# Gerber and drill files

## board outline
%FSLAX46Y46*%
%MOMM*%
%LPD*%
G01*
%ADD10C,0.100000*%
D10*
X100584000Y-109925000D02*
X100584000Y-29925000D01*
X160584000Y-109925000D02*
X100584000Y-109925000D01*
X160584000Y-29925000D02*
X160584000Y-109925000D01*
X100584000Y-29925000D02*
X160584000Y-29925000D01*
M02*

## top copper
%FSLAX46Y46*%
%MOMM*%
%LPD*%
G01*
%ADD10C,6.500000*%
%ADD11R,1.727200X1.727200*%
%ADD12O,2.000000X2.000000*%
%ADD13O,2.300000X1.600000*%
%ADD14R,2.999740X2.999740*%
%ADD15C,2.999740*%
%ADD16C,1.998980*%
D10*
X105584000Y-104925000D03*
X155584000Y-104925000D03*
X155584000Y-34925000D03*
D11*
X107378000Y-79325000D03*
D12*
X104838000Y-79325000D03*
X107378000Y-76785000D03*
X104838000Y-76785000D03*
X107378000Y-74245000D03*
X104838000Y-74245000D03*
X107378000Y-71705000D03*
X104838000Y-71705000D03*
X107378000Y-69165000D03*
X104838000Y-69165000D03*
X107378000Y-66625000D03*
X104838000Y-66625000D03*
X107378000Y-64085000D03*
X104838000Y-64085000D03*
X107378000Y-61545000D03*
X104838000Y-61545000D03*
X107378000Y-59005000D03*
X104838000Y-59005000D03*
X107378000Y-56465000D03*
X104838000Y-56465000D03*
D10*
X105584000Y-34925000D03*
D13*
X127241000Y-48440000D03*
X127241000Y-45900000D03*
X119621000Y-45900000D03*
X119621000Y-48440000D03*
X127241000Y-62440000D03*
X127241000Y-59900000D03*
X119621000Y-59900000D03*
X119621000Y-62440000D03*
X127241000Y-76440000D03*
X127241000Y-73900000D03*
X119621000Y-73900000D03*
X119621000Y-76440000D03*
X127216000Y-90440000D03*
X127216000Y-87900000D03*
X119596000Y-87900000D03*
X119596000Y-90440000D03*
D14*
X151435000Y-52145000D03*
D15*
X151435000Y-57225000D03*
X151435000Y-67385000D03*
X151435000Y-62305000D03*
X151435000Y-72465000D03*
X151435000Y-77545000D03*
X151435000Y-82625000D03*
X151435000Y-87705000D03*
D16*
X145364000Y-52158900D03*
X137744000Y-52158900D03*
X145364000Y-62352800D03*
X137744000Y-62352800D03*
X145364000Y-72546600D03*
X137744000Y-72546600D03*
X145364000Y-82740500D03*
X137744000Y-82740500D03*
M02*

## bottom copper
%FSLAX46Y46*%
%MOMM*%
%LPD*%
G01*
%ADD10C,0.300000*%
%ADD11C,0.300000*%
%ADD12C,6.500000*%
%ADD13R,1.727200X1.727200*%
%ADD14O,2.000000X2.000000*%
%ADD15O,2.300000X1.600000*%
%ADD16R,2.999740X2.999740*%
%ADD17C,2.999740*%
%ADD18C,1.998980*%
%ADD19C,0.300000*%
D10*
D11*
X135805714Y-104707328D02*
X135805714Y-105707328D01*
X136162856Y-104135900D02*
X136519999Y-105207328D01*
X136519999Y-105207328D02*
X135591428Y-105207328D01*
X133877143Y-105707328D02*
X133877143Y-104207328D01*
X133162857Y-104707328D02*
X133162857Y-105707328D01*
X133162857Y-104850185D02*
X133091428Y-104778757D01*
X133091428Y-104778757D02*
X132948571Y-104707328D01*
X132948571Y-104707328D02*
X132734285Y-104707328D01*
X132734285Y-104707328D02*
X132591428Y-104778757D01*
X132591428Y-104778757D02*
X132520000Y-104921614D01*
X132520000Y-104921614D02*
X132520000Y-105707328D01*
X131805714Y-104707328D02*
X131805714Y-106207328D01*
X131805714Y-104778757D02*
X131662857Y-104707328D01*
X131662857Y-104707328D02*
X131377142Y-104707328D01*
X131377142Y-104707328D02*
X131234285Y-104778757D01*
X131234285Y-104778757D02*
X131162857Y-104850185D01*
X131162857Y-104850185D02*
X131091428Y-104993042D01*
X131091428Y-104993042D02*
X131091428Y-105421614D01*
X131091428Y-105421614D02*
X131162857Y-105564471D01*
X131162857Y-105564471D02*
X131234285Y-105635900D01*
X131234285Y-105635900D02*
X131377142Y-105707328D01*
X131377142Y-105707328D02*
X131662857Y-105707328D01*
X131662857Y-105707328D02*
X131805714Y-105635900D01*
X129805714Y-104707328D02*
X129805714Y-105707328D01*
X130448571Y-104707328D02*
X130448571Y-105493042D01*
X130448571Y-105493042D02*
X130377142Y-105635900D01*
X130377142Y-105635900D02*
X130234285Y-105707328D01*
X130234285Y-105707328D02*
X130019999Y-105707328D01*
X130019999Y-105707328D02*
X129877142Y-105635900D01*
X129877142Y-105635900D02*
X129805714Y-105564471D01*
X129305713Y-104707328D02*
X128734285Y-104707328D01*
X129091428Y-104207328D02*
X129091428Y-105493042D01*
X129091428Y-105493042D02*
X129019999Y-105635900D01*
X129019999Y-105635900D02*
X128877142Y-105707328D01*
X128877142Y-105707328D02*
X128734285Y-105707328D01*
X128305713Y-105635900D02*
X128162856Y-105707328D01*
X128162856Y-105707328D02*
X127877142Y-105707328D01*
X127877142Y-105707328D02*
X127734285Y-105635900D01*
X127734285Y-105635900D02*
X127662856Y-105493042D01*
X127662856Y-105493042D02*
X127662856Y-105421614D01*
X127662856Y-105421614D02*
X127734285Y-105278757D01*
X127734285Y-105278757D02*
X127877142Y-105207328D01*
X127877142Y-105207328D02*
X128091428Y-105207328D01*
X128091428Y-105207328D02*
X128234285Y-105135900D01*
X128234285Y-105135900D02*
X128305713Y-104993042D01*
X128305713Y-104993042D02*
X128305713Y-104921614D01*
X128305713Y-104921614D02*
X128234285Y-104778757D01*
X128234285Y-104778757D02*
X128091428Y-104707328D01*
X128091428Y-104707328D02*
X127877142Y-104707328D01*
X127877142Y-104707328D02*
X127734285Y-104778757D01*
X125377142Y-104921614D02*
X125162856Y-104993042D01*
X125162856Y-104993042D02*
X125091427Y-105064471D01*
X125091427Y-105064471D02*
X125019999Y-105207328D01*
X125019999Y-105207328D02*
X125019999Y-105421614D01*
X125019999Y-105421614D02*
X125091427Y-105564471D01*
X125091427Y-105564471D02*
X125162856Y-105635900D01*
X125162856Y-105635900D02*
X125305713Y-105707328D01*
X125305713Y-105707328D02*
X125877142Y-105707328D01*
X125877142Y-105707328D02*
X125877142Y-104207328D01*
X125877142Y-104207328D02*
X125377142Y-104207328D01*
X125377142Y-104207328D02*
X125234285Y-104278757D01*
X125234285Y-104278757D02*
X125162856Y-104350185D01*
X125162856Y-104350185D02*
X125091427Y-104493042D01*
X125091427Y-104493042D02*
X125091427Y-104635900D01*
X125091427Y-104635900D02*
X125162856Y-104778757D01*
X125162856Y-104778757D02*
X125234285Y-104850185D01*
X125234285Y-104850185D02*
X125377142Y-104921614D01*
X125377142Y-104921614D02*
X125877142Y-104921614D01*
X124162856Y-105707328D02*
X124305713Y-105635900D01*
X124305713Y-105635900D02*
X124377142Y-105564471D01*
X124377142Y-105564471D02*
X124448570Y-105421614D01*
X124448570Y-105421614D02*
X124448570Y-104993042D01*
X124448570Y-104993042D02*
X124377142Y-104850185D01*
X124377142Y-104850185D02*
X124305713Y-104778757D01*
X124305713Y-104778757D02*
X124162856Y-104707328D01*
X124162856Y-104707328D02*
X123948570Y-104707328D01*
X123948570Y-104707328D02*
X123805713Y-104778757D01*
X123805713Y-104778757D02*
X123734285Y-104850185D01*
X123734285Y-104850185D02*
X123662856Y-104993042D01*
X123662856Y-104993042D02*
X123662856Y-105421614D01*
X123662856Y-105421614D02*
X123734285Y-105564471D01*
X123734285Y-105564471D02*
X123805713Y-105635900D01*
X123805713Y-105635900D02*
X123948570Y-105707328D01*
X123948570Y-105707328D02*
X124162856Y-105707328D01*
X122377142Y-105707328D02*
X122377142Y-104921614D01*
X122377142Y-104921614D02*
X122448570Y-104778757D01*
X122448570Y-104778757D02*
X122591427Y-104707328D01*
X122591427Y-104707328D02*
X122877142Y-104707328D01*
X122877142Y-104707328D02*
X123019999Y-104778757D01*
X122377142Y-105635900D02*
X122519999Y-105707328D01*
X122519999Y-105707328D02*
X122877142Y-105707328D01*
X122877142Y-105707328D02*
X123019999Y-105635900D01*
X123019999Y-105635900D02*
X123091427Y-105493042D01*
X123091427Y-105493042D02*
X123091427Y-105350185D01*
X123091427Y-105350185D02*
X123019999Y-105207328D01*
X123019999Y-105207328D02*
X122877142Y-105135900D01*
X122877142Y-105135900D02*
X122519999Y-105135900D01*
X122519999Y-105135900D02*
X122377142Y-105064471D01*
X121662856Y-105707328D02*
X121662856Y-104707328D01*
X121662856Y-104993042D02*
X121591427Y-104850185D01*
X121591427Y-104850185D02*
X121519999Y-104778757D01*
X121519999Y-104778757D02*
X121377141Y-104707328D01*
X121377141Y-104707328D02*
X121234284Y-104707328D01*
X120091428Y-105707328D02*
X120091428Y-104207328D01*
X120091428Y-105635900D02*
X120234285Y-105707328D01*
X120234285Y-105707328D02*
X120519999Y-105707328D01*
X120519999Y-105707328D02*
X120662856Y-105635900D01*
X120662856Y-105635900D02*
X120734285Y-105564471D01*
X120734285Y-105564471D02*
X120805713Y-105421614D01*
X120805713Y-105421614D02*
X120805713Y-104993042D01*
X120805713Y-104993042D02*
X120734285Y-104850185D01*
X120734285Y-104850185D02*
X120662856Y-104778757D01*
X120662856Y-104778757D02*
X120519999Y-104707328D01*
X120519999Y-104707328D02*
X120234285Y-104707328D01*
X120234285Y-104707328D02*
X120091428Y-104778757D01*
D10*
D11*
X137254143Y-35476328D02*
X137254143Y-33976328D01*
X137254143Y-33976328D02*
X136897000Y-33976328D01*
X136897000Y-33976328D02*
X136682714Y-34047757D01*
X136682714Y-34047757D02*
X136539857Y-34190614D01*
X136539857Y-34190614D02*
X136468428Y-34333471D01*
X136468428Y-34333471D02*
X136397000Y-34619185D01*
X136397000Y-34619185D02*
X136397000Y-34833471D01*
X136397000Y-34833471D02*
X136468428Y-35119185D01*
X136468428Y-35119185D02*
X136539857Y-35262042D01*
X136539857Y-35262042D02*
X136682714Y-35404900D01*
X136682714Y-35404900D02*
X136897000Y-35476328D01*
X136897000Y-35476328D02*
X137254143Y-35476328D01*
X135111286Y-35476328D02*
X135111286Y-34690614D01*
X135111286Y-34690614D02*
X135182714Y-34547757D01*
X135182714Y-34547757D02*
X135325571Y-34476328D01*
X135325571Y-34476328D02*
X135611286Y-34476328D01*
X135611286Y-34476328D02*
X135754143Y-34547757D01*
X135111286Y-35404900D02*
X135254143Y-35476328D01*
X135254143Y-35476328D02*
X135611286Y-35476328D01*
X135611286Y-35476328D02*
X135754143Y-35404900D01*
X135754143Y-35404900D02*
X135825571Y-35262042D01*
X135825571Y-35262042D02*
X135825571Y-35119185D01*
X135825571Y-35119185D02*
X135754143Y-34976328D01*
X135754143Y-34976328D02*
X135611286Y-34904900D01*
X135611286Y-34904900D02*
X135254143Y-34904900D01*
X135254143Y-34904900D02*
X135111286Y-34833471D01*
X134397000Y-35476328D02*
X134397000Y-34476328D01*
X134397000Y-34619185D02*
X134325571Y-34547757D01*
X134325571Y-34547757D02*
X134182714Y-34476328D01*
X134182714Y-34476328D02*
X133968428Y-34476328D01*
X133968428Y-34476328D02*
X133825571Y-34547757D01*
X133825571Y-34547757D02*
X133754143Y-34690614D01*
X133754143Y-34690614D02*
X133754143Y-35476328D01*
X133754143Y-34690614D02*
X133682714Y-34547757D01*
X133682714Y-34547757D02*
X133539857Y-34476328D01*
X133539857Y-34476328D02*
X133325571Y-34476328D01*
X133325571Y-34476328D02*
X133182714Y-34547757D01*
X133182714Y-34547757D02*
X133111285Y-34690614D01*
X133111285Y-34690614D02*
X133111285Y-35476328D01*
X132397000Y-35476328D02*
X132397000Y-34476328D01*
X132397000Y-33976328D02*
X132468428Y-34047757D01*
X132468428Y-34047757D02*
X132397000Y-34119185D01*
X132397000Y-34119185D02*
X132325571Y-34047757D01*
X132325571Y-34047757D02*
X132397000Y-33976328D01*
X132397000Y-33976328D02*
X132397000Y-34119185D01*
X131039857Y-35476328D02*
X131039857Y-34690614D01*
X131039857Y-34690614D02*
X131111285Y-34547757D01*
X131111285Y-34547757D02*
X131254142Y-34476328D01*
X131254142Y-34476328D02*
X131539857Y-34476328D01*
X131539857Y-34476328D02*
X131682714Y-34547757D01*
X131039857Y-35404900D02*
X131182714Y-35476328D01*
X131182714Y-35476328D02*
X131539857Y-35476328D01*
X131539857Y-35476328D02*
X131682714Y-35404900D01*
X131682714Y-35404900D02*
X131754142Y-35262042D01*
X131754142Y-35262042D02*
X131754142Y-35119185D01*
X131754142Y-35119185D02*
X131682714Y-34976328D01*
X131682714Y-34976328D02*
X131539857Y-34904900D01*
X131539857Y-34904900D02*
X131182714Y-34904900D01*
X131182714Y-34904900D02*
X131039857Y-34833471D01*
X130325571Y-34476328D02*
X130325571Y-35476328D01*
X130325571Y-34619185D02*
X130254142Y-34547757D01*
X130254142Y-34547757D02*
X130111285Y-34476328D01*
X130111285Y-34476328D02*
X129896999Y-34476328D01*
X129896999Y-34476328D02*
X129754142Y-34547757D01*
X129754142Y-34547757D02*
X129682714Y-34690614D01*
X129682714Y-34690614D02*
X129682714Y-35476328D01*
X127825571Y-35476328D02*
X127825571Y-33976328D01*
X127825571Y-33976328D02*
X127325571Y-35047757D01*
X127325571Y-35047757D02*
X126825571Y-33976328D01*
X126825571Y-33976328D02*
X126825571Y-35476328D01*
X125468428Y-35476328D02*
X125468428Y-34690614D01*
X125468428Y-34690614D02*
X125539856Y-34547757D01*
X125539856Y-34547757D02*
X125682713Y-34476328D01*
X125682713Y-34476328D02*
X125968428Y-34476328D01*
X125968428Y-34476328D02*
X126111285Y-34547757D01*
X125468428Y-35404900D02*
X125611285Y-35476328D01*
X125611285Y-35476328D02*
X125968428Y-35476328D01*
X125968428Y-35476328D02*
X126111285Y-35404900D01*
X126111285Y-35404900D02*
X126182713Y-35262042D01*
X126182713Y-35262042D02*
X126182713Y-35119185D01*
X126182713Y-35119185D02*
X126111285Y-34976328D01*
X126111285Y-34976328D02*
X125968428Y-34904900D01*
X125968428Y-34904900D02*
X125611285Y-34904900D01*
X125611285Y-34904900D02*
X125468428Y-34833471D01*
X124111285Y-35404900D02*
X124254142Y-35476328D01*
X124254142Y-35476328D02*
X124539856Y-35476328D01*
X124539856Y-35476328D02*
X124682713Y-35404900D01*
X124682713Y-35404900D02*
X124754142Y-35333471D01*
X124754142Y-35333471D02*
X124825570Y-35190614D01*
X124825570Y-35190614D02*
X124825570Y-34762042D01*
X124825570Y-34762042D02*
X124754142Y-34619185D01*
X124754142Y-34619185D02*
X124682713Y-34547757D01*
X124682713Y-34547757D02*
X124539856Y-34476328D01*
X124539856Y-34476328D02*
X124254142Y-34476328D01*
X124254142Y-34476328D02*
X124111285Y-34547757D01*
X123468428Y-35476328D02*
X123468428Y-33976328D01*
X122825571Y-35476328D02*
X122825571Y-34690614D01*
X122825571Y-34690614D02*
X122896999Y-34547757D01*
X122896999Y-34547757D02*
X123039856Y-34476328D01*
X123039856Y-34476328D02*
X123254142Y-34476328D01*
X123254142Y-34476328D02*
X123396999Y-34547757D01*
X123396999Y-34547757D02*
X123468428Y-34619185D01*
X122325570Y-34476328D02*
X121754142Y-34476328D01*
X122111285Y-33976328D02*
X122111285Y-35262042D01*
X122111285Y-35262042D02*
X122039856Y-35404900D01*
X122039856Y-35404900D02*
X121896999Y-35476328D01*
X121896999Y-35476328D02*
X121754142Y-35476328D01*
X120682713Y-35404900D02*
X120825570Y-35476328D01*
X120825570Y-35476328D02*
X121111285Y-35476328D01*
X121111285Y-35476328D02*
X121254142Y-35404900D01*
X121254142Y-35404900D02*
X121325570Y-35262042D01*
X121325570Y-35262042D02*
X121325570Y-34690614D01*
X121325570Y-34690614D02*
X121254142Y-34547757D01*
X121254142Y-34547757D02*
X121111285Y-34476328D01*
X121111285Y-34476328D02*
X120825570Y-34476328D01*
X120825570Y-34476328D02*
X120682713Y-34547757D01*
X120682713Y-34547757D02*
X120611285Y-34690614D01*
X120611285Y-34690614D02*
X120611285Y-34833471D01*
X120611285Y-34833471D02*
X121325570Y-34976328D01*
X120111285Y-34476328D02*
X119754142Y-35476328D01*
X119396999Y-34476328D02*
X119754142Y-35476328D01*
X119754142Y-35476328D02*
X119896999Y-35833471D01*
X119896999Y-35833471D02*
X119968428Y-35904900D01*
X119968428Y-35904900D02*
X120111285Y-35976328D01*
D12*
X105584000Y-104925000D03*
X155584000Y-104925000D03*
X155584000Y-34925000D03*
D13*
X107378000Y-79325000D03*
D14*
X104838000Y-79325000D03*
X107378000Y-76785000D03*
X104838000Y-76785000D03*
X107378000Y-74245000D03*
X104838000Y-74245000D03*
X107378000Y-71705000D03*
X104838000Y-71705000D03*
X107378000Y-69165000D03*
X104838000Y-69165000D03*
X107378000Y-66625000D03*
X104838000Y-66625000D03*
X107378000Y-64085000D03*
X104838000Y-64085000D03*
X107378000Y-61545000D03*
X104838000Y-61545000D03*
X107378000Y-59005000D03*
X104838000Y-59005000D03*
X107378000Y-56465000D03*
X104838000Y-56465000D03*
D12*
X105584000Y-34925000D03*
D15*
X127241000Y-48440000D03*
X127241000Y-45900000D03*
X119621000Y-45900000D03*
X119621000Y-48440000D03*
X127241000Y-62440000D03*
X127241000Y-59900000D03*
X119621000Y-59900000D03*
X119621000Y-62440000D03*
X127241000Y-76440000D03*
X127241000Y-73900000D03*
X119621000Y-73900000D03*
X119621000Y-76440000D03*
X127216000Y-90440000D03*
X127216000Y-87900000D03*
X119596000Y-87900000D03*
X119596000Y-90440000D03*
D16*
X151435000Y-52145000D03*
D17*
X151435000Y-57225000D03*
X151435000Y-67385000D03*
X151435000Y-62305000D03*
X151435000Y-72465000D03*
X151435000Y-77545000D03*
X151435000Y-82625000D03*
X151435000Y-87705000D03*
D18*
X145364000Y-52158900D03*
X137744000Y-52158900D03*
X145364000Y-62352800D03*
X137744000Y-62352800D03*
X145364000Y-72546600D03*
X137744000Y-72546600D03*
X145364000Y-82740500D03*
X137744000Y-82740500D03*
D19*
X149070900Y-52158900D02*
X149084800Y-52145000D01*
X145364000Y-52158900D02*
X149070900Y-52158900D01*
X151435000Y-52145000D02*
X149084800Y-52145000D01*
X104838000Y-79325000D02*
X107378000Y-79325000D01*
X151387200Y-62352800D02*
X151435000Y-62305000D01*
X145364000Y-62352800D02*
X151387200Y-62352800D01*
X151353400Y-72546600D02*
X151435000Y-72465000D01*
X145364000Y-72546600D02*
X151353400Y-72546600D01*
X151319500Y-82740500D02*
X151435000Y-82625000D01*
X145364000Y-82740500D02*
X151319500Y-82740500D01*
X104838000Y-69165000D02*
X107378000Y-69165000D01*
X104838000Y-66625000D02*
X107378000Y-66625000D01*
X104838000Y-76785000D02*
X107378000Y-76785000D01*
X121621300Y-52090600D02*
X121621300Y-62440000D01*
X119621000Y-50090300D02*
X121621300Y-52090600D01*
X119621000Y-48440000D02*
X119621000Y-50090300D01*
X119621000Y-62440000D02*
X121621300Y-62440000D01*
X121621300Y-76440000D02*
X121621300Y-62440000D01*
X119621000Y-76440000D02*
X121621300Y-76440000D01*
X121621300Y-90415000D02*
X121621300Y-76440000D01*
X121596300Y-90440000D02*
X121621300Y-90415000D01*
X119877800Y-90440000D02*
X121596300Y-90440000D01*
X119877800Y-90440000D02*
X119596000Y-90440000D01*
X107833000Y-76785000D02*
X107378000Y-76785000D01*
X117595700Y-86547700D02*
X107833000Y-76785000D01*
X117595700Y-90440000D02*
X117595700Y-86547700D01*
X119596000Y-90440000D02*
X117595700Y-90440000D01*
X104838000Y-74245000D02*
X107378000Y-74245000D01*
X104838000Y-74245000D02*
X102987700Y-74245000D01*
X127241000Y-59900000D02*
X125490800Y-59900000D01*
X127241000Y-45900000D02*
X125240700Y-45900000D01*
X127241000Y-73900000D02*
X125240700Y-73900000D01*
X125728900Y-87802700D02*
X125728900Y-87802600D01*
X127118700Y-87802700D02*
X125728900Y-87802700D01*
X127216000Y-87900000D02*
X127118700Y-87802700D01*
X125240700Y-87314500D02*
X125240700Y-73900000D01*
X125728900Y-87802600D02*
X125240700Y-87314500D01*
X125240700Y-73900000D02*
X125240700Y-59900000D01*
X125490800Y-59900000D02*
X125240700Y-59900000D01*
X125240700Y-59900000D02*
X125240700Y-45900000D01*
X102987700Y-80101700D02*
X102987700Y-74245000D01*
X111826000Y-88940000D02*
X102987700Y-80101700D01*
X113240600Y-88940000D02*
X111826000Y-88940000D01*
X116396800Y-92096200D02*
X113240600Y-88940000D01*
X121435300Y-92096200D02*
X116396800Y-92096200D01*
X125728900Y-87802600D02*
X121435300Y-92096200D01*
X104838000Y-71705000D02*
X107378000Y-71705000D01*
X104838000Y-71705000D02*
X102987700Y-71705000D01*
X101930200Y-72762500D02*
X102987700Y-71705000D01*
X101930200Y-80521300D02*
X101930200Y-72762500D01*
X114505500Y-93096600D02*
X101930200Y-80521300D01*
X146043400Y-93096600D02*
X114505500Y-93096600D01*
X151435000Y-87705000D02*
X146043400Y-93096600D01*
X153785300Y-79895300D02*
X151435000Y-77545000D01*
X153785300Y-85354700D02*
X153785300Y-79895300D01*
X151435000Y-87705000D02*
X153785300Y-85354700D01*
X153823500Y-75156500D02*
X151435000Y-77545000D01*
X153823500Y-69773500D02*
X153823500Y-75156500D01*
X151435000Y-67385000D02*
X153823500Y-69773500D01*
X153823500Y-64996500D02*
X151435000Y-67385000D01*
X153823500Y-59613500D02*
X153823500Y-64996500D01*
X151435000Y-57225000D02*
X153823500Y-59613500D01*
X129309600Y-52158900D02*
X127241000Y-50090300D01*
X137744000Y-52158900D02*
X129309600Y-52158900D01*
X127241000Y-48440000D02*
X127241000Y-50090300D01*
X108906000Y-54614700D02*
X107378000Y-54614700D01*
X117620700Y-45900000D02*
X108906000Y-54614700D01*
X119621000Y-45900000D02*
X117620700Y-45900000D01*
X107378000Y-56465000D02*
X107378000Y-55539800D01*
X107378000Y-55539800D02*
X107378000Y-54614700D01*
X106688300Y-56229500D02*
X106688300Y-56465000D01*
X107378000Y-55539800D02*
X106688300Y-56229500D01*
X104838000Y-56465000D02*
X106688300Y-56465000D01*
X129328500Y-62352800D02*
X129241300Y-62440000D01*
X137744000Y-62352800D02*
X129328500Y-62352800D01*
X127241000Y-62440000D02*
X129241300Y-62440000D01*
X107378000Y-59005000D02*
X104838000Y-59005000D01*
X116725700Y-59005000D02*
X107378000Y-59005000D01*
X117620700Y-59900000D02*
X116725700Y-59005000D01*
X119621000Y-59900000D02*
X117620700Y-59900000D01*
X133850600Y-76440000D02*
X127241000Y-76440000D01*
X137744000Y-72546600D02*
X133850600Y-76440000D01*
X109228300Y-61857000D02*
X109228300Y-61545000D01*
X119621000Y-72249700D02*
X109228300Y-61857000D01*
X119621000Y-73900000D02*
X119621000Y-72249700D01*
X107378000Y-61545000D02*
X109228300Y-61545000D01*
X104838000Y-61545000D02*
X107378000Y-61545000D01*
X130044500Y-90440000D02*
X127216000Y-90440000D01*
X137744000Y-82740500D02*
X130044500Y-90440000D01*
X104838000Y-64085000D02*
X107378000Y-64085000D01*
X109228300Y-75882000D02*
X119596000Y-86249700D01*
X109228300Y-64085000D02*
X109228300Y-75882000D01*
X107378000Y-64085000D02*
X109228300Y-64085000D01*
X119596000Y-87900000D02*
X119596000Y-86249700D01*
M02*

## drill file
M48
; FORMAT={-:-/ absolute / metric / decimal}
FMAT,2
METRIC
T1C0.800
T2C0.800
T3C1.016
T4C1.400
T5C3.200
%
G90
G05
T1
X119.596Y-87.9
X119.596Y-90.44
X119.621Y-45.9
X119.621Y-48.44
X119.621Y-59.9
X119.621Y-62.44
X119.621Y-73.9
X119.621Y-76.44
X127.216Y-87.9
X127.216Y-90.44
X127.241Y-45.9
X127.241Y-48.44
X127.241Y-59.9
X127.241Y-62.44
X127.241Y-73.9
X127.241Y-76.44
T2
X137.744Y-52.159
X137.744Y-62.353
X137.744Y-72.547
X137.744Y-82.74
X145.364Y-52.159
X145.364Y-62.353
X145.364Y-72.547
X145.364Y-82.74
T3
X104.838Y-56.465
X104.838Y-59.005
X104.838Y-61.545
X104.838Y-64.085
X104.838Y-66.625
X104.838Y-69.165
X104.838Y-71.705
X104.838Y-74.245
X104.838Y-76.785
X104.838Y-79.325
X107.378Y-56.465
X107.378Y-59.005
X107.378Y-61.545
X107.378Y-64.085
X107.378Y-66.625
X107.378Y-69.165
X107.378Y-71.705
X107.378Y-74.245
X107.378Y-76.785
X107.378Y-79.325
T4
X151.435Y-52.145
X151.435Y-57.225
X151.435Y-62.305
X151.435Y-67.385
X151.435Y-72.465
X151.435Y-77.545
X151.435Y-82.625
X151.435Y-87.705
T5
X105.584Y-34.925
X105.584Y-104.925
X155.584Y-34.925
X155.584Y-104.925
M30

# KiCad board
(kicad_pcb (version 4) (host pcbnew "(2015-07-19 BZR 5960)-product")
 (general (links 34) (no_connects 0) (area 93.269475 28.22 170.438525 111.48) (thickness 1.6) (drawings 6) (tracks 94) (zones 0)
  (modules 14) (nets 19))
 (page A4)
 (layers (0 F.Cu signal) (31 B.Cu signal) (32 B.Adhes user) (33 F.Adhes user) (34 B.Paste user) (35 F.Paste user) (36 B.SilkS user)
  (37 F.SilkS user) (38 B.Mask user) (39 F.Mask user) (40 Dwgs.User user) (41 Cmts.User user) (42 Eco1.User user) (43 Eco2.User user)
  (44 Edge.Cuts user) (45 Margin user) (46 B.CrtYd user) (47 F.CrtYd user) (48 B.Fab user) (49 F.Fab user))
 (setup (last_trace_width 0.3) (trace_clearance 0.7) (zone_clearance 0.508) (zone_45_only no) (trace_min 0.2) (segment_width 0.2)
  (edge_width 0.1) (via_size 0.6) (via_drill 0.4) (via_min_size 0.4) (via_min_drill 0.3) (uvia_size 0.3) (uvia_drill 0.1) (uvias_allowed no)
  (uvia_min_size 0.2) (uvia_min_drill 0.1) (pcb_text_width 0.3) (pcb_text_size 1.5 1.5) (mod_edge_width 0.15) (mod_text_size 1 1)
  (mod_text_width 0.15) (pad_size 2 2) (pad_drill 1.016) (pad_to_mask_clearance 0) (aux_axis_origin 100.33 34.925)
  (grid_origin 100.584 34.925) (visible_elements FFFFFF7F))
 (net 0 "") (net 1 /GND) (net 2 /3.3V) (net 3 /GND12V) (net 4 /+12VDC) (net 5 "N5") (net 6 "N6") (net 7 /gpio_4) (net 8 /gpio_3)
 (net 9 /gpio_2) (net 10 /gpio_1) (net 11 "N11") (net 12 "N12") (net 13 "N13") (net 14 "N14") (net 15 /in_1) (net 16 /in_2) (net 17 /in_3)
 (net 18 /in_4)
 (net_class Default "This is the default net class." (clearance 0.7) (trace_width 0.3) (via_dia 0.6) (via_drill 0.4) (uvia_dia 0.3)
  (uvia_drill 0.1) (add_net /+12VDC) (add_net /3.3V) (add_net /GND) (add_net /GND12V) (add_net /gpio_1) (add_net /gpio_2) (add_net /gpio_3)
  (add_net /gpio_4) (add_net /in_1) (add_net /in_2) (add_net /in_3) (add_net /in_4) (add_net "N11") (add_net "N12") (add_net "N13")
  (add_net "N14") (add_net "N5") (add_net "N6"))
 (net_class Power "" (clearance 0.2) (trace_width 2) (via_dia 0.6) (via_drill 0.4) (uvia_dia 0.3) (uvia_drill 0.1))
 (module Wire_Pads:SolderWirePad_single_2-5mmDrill (layer F.Cu) (at 105.584 104.925)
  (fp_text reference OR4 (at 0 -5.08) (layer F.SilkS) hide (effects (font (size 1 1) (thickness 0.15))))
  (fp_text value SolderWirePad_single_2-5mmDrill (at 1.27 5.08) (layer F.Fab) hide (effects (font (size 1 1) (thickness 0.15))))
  (pad 1 thru_hole circle (at 0 0) (size 6.5 6.5) (drill 3.2) (layers *.Cu *.Mask F.SilkS)))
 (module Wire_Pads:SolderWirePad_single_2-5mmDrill (layer F.Cu) (at 155.584 104.925)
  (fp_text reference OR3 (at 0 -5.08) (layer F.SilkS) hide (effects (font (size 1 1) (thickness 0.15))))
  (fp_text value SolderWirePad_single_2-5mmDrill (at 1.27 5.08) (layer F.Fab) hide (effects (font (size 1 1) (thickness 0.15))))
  (pad 1 thru_hole circle (at 0 0) (size 6.5 6.5) (drill 3.2) (layers *.Cu *.Mask F.SilkS)))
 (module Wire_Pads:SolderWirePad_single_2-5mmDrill (layer F.Cu) (at 155.584 34.925)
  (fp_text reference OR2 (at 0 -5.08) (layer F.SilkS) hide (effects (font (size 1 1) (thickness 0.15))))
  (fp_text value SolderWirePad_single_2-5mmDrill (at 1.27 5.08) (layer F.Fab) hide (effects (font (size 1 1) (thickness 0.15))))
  (pad 1 thru_hole circle (at 0 0) (size 6.5 6.5) (drill 3.2) (layers *.Cu *.Mask F.SilkS)))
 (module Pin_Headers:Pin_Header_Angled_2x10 (layer F.Cu) (at 107.378 79.325 180)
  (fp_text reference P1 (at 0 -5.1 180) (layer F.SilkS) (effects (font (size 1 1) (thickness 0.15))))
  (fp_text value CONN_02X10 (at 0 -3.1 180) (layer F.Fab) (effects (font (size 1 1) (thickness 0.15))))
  (pad 1 thru_hole rect (at 0 0 180) (size 1.7272 1.7272) (drill 1.016) (layers *.Cu *.Mask F.SilkS) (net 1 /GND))
  (pad 2 thru_hole oval (at 2.54 0 180) (size 2 2) (drill 1.016) (layers *.Cu *.Mask F.SilkS) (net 1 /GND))
  (pad 3 thru_hole oval (at 0 2.54 180) (size 2 2) (drill 1.016) (layers *.Cu *.Mask F.SilkS) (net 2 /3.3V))
  (pad 4 thru_hole oval (at 2.54 2.54 180) (size 2 2) (drill 1.016) (layers *.Cu *.Mask F.SilkS) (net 2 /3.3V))
  (pad 5 thru_hole oval (at 0 5.08 180) (size 2 2) (drill 1.016) (layers *.Cu *.Mask F.SilkS) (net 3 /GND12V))
  (pad 6 thru_hole oval (at 2.54 5.08 180) (size 2 2) (drill 1.016) (layers *.Cu *.Mask F.SilkS) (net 3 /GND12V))
  (pad 7 thru_hole oval (at 0 7.62 180) (size 2 2) (drill 1.016) (layers *.Cu *.Mask F.SilkS) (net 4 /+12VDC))
  (pad 8 thru_hole oval (at 2.54 7.62 180) (size 2 2) (drill 1.016) (layers *.Cu *.Mask F.SilkS) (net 4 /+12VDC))
  (pad 9 thru_hole oval (at 0 10.16 180) (size 2 2) (drill 1.016) (layers *.Cu *.Mask F.SilkS) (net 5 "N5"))
  (pad 10 thru_hole oval (at 2.54 10.16 180) (size 2 2) (drill 1.016) (layers *.Cu *.Mask F.SilkS) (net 5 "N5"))
  (pad 11 thru_hole oval (at 0 12.7 180) (size 2 2) (drill 1.016) (layers *.Cu *.Mask F.SilkS) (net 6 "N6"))
  (pad 12 thru_hole oval (at 2.54 12.7 180) (size 2 2) (drill 1.016) (layers *.Cu *.Mask F.SilkS) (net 6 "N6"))
  (pad 13 thru_hole oval (at 0 15.24 180) (size 2 2) (drill 1.016) (layers *.Cu *.Mask F.SilkS) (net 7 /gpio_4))
  (pad 14 thru_hole oval (at 2.54 15.24 180) (size 2 2) (drill 1.016) (layers *.Cu *.Mask F.SilkS) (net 7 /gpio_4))
  (pad 15 thru_hole oval (at 0 17.78 180) (size 2 2) (drill 1.016) (layers *.Cu *.Mask F.SilkS) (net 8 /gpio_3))
  (pad 16 thru_hole oval (at 2.54 17.78 180) (size 2 2) (drill 1.016) (layers *.Cu *.Mask F.SilkS) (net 8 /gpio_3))
  (pad 17 thru_hole oval (at 0 20.32 180) (size 2 2) (drill 1.016) (layers *.Cu *.Mask F.SilkS) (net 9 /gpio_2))
  (pad 18 thru_hole oval (at 2.54 20.32 180) (size 2 2) (drill 1.016) (layers *.Cu *.Mask F.SilkS) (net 9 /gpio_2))
  (pad 19 thru_hole oval (at 0 22.86 180) (size 2 2) (drill 1.016) (layers *.Cu *.Mask F.SilkS) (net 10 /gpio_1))
  (pad 20 thru_hole oval (at 2.54 22.86 180) (size 2 2) (drill 1.016) (layers *.Cu *.Mask F.SilkS) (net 10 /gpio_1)))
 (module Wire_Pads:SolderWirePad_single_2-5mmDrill (layer F.Cu) (at 105.584 34.925)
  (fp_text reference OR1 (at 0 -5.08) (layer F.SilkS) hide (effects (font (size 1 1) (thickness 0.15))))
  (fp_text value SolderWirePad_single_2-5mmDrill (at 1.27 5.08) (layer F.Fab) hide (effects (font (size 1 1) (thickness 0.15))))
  (pad 1 thru_hole circle (at 0 0) (size 6.5 6.5) (drill 3.2) (layers *.Cu *.Mask F.SilkS)))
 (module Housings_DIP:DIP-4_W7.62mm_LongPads (layer F.Cu) (at 127.241 48.44 180)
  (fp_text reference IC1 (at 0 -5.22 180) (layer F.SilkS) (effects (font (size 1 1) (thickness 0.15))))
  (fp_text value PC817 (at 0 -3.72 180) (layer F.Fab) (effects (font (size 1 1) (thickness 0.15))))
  (pad 1 thru_hole oval (at 0 0 180) (size 2.3 1.6) (drill 0.8) (layers *.Cu *.Mask F.SilkS) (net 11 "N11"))
  (pad 2 thru_hole oval (at 0 2.54 180) (size 2.3 1.6) (drill 0.8) (layers *.Cu *.Mask F.SilkS) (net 3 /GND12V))
  (pad 3 thru_hole oval (at 7.62 2.54 180) (size 2.3 1.6) (drill 0.8) (layers *.Cu *.Mask F.SilkS) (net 10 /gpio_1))
  (pad 4 thru_hole oval (at 7.62 0 180) (size 2.3 1.6) (drill 0.8) (layers *.Cu *.Mask F.SilkS) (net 2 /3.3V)))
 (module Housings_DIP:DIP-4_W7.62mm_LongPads (layer F.Cu) (at 127.241 62.44 180)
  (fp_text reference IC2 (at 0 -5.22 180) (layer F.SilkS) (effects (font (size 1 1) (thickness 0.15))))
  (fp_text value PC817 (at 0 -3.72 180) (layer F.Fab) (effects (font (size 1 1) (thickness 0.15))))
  (pad 1 thru_hole oval (at 0 0 180) (size 2.3 1.6) (drill 0.8) (layers *.Cu *.Mask F.SilkS) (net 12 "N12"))
  (pad 2 thru_hole oval (at 0 2.54 180) (size 2.3 1.6) (drill 0.8) (layers *.Cu *.Mask F.SilkS) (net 3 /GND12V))
  (pad 3 thru_hole oval (at 7.62 2.54 180) (size 2.3 1.6) (drill 0.8) (layers *.Cu *.Mask F.SilkS) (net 9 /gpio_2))
  (pad 4 thru_hole oval (at 7.62 0 180) (size 2.3 1.6) (drill 0.8) (layers *.Cu *.Mask F.SilkS) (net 2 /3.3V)))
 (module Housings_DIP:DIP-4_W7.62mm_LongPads (layer F.Cu) (at 127.241 76.44 180)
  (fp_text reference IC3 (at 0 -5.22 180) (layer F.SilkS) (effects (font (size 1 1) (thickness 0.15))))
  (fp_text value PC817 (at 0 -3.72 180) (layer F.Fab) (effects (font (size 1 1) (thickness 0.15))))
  (pad 1 thru_hole oval (at 0 0 180) (size 2.3 1.6) (drill 0.8) (layers *.Cu *.Mask F.SilkS) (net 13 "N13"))
  (pad 2 thru_hole oval (at 0 2.54 180) (size 2.3 1.6) (drill 0.8) (layers *.Cu *.Mask F.SilkS) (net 3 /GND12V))
  (pad 3 thru_hole oval (at 7.62 2.54 180) (size 2.3 1.6) (drill 0.8) (layers *.Cu *.Mask F.SilkS) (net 8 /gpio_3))
  (pad 4 thru_hole oval (at 7.62 0 180) (size 2.3 1.6) (drill 0.8) (layers *.Cu *.Mask F.SilkS) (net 2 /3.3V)))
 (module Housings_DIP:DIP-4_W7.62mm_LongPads (layer F.Cu) (at 127.216 90.44 180)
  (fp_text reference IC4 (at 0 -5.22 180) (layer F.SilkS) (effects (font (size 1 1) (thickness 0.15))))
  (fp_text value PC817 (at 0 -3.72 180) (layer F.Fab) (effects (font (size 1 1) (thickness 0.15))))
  (pad 1 thru_hole oval (at 0 0 180) (size 2.3 1.6) (drill 0.8) (layers *.Cu *.Mask F.SilkS) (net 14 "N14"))
  (pad 2 thru_hole oval (at 0 2.54 180) (size 2.3 1.6) (drill 0.8) (layers *.Cu *.Mask F.SilkS) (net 3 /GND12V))
  (pad 3 thru_hole oval (at 7.62 2.54 180) (size 2.3 1.6) (drill 0.8) (layers *.Cu *.Mask F.SilkS) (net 7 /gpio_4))
  (pad 4 thru_hole oval (at 7.62 0 180) (size 2.3 1.6) (drill 0.8) (layers *.Cu *.Mask F.SilkS) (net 2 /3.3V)))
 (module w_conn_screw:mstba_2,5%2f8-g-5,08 (layer F.Cu) (at 151.435 69.925 270)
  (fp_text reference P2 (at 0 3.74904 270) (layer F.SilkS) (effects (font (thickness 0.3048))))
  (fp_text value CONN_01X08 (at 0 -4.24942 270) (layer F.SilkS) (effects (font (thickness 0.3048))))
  (pad 1 thru_hole rect (at -17.78 0 270) (size 2.99974 2.99974) (drill 1.39954) (layers *.Cu *.Mask F.SilkS) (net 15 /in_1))
  (pad 2 thru_hole circle (at -12.7 0 270) (size 2.99974 2.99974) (drill 1.39954) (layers *.Cu *.Mask F.SilkS) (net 4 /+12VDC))
  (pad 4 thru_hole circle (at -2.54 0 270) (size 2.99974 2.99974) (drill 1.39954) (layers *.Cu *.Mask F.SilkS) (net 4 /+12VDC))
  (pad 3 thru_hole circle (at -7.62 0 270) (size 2.99974 2.99974) (drill 1.39954) (layers *.Cu *.Mask F.SilkS) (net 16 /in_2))
  (pad 5 thru_hole circle (at 2.54 0 270) (size 2.99974 2.99974) (drill 1.39954) (layers *.Cu *.Mask F.SilkS) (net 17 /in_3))
  (pad 6 thru_hole circle (at 7.62 0 270) (size 2.99974 2.99974) (drill 1.39954) (layers *.Cu *.Mask F.SilkS) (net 4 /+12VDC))
  (pad 7 thru_hole circle (at 12.7 0 270) (size 2.99974 2.99974) (drill 1.39954) (layers *.Cu *.Mask F.SilkS) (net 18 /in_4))
  (pad 8 thru_hole circle (at 17.78 0 270) (size 2.99974 2.99974) (drill 1.39954) (layers *.Cu *.Mask F.SilkS) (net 4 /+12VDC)))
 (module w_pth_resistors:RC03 (layer F.Cu) (at 141.554 52.1589 180) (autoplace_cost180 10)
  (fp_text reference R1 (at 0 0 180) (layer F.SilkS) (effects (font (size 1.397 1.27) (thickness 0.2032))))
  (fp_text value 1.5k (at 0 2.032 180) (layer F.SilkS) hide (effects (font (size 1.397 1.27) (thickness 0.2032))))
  (pad 1 thru_hole circle (at -3.81 0 180) (size 1.99898 1.99898) (drill 0.8001) (layers *.Cu *.Mask F.SilkS) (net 15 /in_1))
  (pad 2 thru_hole circle (at 3.81 0 180) (size 1.99898 1.99898) (drill 0.8001) (layers *.Cu *.Mask F.SilkS) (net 11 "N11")))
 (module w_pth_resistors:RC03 (layer F.Cu) (at 141.554 62.3528 180) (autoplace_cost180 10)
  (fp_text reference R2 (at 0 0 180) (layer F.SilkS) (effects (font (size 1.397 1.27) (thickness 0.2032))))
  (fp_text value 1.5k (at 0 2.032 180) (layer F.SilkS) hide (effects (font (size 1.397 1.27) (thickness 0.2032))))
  (pad 1 thru_hole circle (at -3.81 0 180) (size 1.99898 1.99898) (drill 0.8001) (layers *.Cu *.Mask F.SilkS) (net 16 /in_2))
  (pad 2 thru_hole circle (at 3.81 0 180) (size 1.99898 1.99898) (drill 0.8001) (layers *.Cu *.Mask F.SilkS) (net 12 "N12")))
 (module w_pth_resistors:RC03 (layer F.Cu) (at 141.554 72.5466 180) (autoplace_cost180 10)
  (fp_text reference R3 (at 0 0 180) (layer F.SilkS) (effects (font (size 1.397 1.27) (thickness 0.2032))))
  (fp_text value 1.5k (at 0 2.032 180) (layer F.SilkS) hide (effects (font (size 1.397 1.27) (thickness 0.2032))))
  (pad 1 thru_hole circle (at -3.81 0 180) (size 1.99898 1.99898) (drill 0.8001) (layers *.Cu *.Mask F.SilkS) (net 17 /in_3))
  (pad 2 thru_hole circle (at 3.81 0 180) (size 1.99898 1.99898) (drill 0.8001) (layers *.Cu *.Mask F.SilkS) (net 13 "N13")))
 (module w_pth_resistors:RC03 (layer F.Cu) (at 141.554 82.7405 180) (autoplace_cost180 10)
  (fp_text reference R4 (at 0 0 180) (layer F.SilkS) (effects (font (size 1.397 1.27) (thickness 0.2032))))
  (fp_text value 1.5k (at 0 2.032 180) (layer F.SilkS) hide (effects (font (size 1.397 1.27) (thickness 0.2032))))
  (pad 1 thru_hole circle (at -3.81 0 180) (size 1.99898 1.99898) (drill 0.8001) (layers *.Cu *.Mask F.SilkS) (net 18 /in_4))
  (pad 2 thru_hole circle (at 3.81 0 180) (size 1.99898 1.99898) (drill 0.8001) (layers *.Cu *.Mask F.SilkS) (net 14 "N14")))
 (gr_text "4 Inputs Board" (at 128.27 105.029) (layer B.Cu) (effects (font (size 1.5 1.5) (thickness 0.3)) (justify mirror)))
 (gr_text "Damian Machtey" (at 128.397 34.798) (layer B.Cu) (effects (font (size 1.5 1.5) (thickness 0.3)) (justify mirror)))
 (gr_line (start 100.584 109.925) (end 100.584 29.925) (angle 90) (layer Edge.Cuts) (width 0.1))
 (gr_line (start 160.584 109.925) (end 100.584 109.925) (angle 90) (layer Edge.Cuts) (width 0.1))
 (gr_line (start 160.584 29.925) (end 160.584 109.925) (angle 90) (layer Edge.Cuts) (width 0.1))
 (gr_line (start 100.584 29.925) (end 160.584 29.925) (angle 90) (layer Edge.Cuts) (width 0.1))
 (segment (start 149.0709 52.1589) (end 149.0848 52.145) (width 0.3) (layer B.Cu) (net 15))
 (segment (start 145.364 52.1589) (end 149.0709 52.1589) (width 0.3) (layer B.Cu) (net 15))
 (segment (start 151.435 52.145) (end 149.0848 52.145) (width 0.3) (layer B.Cu) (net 15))
 (segment (start 104.838 79.325) (end 107.378 79.325) (width 0.3) (layer B.Cu) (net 1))
 (segment (start 151.3872 62.3528) (end 151.435 62.305) (width 0.3) (layer B.Cu) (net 16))
 (segment (start 145.364 62.3528) (end 151.3872 62.3528) (width 0.3) (layer B.Cu) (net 16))
 (segment (start 151.3534 72.5466) (end 151.435 72.465) (width 0.3) (layer B.Cu) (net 17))
 (segment (start 145.364 72.5466) (end 151.3534 72.5466) (width 0.3) (layer B.Cu) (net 17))
 (segment (start 151.3195 82.7405) (end 151.435 82.625) (width 0.3) (layer B.Cu) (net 18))
 (segment (start 145.364 82.7405) (end 151.3195 82.7405) (width 0.3) (layer B.Cu) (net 18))
 (segment (start 104.838 69.165) (end 107.378 69.165) (width 0.3) (layer B.Cu) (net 5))
 (segment (start 104.838 66.625) (end 107.378 66.625) (width 0.3) (layer B.Cu) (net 6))
 (segment (start 104.838 76.785) (end 107.378 76.785) (width 0.3) (layer B.Cu) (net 2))
 (segment (start 121.6213 52.0906) (end 121.6213 62.44) (width 0.3) (layer B.Cu) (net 2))
 (segment (start 119.621 50.0903) (end 121.6213 52.0906) (width 0.3) (layer B.Cu) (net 2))
 (segment (start 119.621 48.44) (end 119.621 50.0903) (width 0.3) (layer B.Cu) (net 2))
 (segment (start 119.621 62.44) (end 121.6213 62.44) (width 0.3) (layer B.Cu) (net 2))
 (segment (start 121.6213 76.44) (end 121.6213 62.44) (width 0.3) (layer B.Cu) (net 2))
 (segment (start 119.621 76.44) (end 121.6213 76.44) (width 0.3) (layer B.Cu) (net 2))
 (segment (start 121.6213 90.415) (end 121.6213 76.44) (width 0.3) (layer B.Cu) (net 2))
 (segment (start 121.5963 90.44) (end 121.6213 90.415) (width 0.3) (layer B.Cu) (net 2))
 (segment (start 119.8778 90.44) (end 121.5963 90.44) (width 0.3) (layer B.Cu) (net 2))
 (segment (start 119.8778 90.44) (end 119.596 90.44) (width 0.3) (layer B.Cu) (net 2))
 (segment (start 107.833 76.785) (end 107.378 76.785) (width 0.3) (layer B.Cu) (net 2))
 (segment (start 117.5957 86.5477) (end 107.833 76.785) (width 0.3) (layer B.Cu) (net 2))
 (segment (start 117.5957 90.44) (end 117.5957 86.5477) (width 0.3) (layer B.Cu) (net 2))
 (segment (start 119.596 90.44) (end 117.5957 90.44) (width 0.3) (layer B.Cu) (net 2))
 (segment (start 104.838 74.245) (end 107.378 74.245) (width 0.3) (layer B.Cu) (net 3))
 (segment (start 104.838 74.245) (end 102.9877 74.245) (width 0.3) (layer B.Cu) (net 3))
 (segment (start 127.241 59.9) (end 125.4908 59.9) (width 0.3) (layer B.Cu) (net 3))
 (segment (start 127.241 45.9) (end 125.2407 45.9) (width 0.3) (layer B.Cu) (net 3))
 (segment (start 127.241 73.9) (end 125.2407 73.9) (width 0.3) (layer B.Cu) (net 3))
 (segment (start 125.7289 87.8027) (end 125.7289 87.8026) (width 0.3) (layer B.Cu) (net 3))
 (segment (start 127.1187 87.8027) (end 125.7289 87.8027) (width 0.3) (layer B.Cu) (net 3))
 (segment (start 127.216 87.9) (end 127.1187 87.8027) (width 0.3) (layer B.Cu) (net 3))
 (segment (start 125.2407 87.3145) (end 125.2407 73.9) (width 0.3) (layer B.Cu) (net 3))
 (segment (start 125.7289 87.8026) (end 125.2407 87.3145) (width 0.3) (layer B.Cu) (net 3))
 (segment (start 125.2407 73.9) (end 125.2407 59.9) (width 0.3) (layer B.Cu) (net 3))
 (segment (start 125.4908 59.9) (end 125.2407 59.9) (width 0.3) (layer B.Cu) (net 3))
 (segment (start 125.2407 59.9) (end 125.2407 45.9) (width 0.3) (layer B.Cu) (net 3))
 (segment (start 102.9877 80.1017) (end 102.9877 74.245) (width 0.3) (layer B.Cu) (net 3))
 (segment (start 111.826 88.94) (end 102.9877 80.1017) (width 0.3) (layer B.Cu) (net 3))
 (segment (start 113.2406 88.94) (end 111.826 88.94) (width 0.3) (layer B.Cu) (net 3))
 (segment (start 116.3968 92.0962) (end 113.2406 88.94) (width 0.3) (layer B.Cu) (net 3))
 (segment (start 121.4353 92.0962) (end 116.3968 92.0962) (width 0.3) (layer B.Cu) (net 3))
 (segment (start 125.7289 87.8026) (end 121.4353 92.0962) (width 0.3) (layer B.Cu) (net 3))
 (segment (start 104.838 71.705) (end 107.378 71.705) (width 0.3) (layer B.Cu) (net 4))
 (segment (start 104.838 71.705) (end 102.9877 71.705) (width 0.3) (layer B.Cu) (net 4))
 (segment (start 101.9302 72.7625) (end 102.9877 71.705) (width 0.3) (layer B.Cu) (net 4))
 (segment (start 101.9302 80.5213) (end 101.9302 72.7625) (width 0.3) (layer B.Cu) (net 4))
 (segment (start 114.5055 93.0966) (end 101.9302 80.5213) (width 0.3) (layer B.Cu) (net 4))
 (segment (start 146.0434 93.0966) (end 114.5055 93.0966) (width 0.3) (layer B.Cu) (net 4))
 (segment (start 151.435 87.705) (end 146.0434 93.0966) (width 0.3) (layer B.Cu) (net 4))
 (segment (start 153.7853 79.8953) (end 151.435 77.545) (width 0.3) (layer B.Cu) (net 4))
 (segment (start 153.7853 85.3547) (end 153.7853 79.8953) (width 0.3) (layer B.Cu) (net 4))
 (segment (start 151.435 87.705) (end 153.7853 85.3547) (width 0.3) (layer B.Cu) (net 4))
 (segment (start 153.8235 75.1565) (end 151.435 77.545) (width 0.3) (layer B.Cu) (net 4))
 (segment (start 153.8235 69.7735) (end 153.8235 75.1565) (width 0.3) (layer B.Cu) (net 4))
 (segment (start 151.435 67.385) (end 153.8235 69.7735) (width 0.3) (layer B.Cu) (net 4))
 (segment (start 153.8235 64.9965) (end 151.435 67.385) (width 0.3) (layer B.Cu) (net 4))
 (segment (start 153.8235 59.6135) (end 153.8235 64.9965) (width 0.3) (layer B.Cu) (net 4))
 (segment (start 151.435 57.225) (end 153.8235 59.6135) (width 0.3) (layer B.Cu) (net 4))
 (segment (start 129.3096 52.1589) (end 127.241 50.0903) (width 0.3) (layer B.Cu) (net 11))
 (segment (start 137.744 52.1589) (end 129.3096 52.1589) (width 0.3) (layer B.Cu) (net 11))
 (segment (start 127.241 48.44) (end 127.241 50.0903) (width 0.3) (layer B.Cu) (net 11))
 (segment (start 108.906 54.6147) (end 107.378 54.6147) (width 0.3) (layer B.Cu) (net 10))
 (segment (start 117.6207 45.9) (end 108.906 54.6147) (width 0.3) (layer B.Cu) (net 10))
 (segment (start 119.621 45.9) (end 117.6207 45.9) (width 0.3) (layer B.Cu) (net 10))
 (segment (start 107.378 56.465) (end 107.378 55.5398) (width 0.3) (layer B.Cu) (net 10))
 (segment (start 107.378 55.5398) (end 107.378 54.6147) (width 0.3) (layer B.Cu) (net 10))
 (segment (start 106.6883 56.2295) (end 106.6883 56.465) (width 0.3) (layer B.Cu) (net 10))
 (segment (start 107.378 55.5398) (end 106.6883 56.2295) (width 0.3) (layer B.Cu) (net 10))
 (segment (start 104.838 56.465) (end 106.6883 56.465) (width 0.3) (layer B.Cu) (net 10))
 (segment (start 129.3285 62.3528) (end 129.2413 62.44) (width 0.3) (layer B.Cu) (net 12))
 (segment (start 137.744 62.3528) (end 129.3285 62.3528) (width 0.3) (layer B.Cu) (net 12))
 (segment (start 127.241 62.44) (end 129.2413 62.44) (width 0.3) (layer B.Cu) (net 12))
 (segment (start 107.378 59.005) (end 104.838 59.005) (width 0.3) (layer B.Cu) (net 9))
 (segment (start 116.7257 59.005) (end 107.378 59.005) (width 0.3) (layer B.Cu) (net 9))
 (segment (start 117.6207 59.9) (end 116.7257 59.005) (width 0.3) (layer B.Cu) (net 9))
 (segment (start 119.621 59.9) (end 117.6207 59.9) (width 0.3) (layer B.Cu) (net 9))
 (segment (start 133.8506 76.44) (end 127.241 76.44) (width 0.3) (layer B.Cu) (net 13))
 (segment (start 137.744 72.5466) (end 133.8506 76.44) (width 0.3) (layer B.Cu) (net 13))
 (segment (start 109.2283 61.857) (end 109.2283 61.545) (width 0.3) (layer B.Cu) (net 8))
 (segment (start 119.621 72.2497) (end 109.2283 61.857) (width 0.3) (layer B.Cu) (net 8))
 (segment (start 119.621 73.9) (end 119.621 72.2497) (width 0.3) (layer B.Cu) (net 8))
 (segment (start 107.378 61.545) (end 109.2283 61.545) (width 0.3) (layer B.Cu) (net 8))
 (segment (start 104.838 61.545) (end 107.378 61.545) (width 0.3) (layer B.Cu) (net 8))
 (segment (start 130.0445 90.44) (end 127.216 90.44) (width 0.3) (layer B.Cu) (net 14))
 (segment (start 137.744 82.7405) (end 130.0445 90.44) (width 0.3) (layer B.Cu) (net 14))
 (segment (start 104.838 64.085) (end 107.378 64.085) (width 0.3) (layer B.Cu) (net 7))
 (segment (start 109.2283 75.882) (end 119.596 86.2497) (width 0.3) (layer B.Cu) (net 7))
 (segment (start 109.2283 64.085) (end 109.2283 75.882) (width 0.3) (layer B.Cu) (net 7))
 (segment (start 107.378 64.085) (end 109.2283 64.085) (width 0.3) (layer B.Cu) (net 7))
 (segment (start 119.596 87.9) (end 119.596 86.2497) (width 0.3) (layer B.Cu) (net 7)))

